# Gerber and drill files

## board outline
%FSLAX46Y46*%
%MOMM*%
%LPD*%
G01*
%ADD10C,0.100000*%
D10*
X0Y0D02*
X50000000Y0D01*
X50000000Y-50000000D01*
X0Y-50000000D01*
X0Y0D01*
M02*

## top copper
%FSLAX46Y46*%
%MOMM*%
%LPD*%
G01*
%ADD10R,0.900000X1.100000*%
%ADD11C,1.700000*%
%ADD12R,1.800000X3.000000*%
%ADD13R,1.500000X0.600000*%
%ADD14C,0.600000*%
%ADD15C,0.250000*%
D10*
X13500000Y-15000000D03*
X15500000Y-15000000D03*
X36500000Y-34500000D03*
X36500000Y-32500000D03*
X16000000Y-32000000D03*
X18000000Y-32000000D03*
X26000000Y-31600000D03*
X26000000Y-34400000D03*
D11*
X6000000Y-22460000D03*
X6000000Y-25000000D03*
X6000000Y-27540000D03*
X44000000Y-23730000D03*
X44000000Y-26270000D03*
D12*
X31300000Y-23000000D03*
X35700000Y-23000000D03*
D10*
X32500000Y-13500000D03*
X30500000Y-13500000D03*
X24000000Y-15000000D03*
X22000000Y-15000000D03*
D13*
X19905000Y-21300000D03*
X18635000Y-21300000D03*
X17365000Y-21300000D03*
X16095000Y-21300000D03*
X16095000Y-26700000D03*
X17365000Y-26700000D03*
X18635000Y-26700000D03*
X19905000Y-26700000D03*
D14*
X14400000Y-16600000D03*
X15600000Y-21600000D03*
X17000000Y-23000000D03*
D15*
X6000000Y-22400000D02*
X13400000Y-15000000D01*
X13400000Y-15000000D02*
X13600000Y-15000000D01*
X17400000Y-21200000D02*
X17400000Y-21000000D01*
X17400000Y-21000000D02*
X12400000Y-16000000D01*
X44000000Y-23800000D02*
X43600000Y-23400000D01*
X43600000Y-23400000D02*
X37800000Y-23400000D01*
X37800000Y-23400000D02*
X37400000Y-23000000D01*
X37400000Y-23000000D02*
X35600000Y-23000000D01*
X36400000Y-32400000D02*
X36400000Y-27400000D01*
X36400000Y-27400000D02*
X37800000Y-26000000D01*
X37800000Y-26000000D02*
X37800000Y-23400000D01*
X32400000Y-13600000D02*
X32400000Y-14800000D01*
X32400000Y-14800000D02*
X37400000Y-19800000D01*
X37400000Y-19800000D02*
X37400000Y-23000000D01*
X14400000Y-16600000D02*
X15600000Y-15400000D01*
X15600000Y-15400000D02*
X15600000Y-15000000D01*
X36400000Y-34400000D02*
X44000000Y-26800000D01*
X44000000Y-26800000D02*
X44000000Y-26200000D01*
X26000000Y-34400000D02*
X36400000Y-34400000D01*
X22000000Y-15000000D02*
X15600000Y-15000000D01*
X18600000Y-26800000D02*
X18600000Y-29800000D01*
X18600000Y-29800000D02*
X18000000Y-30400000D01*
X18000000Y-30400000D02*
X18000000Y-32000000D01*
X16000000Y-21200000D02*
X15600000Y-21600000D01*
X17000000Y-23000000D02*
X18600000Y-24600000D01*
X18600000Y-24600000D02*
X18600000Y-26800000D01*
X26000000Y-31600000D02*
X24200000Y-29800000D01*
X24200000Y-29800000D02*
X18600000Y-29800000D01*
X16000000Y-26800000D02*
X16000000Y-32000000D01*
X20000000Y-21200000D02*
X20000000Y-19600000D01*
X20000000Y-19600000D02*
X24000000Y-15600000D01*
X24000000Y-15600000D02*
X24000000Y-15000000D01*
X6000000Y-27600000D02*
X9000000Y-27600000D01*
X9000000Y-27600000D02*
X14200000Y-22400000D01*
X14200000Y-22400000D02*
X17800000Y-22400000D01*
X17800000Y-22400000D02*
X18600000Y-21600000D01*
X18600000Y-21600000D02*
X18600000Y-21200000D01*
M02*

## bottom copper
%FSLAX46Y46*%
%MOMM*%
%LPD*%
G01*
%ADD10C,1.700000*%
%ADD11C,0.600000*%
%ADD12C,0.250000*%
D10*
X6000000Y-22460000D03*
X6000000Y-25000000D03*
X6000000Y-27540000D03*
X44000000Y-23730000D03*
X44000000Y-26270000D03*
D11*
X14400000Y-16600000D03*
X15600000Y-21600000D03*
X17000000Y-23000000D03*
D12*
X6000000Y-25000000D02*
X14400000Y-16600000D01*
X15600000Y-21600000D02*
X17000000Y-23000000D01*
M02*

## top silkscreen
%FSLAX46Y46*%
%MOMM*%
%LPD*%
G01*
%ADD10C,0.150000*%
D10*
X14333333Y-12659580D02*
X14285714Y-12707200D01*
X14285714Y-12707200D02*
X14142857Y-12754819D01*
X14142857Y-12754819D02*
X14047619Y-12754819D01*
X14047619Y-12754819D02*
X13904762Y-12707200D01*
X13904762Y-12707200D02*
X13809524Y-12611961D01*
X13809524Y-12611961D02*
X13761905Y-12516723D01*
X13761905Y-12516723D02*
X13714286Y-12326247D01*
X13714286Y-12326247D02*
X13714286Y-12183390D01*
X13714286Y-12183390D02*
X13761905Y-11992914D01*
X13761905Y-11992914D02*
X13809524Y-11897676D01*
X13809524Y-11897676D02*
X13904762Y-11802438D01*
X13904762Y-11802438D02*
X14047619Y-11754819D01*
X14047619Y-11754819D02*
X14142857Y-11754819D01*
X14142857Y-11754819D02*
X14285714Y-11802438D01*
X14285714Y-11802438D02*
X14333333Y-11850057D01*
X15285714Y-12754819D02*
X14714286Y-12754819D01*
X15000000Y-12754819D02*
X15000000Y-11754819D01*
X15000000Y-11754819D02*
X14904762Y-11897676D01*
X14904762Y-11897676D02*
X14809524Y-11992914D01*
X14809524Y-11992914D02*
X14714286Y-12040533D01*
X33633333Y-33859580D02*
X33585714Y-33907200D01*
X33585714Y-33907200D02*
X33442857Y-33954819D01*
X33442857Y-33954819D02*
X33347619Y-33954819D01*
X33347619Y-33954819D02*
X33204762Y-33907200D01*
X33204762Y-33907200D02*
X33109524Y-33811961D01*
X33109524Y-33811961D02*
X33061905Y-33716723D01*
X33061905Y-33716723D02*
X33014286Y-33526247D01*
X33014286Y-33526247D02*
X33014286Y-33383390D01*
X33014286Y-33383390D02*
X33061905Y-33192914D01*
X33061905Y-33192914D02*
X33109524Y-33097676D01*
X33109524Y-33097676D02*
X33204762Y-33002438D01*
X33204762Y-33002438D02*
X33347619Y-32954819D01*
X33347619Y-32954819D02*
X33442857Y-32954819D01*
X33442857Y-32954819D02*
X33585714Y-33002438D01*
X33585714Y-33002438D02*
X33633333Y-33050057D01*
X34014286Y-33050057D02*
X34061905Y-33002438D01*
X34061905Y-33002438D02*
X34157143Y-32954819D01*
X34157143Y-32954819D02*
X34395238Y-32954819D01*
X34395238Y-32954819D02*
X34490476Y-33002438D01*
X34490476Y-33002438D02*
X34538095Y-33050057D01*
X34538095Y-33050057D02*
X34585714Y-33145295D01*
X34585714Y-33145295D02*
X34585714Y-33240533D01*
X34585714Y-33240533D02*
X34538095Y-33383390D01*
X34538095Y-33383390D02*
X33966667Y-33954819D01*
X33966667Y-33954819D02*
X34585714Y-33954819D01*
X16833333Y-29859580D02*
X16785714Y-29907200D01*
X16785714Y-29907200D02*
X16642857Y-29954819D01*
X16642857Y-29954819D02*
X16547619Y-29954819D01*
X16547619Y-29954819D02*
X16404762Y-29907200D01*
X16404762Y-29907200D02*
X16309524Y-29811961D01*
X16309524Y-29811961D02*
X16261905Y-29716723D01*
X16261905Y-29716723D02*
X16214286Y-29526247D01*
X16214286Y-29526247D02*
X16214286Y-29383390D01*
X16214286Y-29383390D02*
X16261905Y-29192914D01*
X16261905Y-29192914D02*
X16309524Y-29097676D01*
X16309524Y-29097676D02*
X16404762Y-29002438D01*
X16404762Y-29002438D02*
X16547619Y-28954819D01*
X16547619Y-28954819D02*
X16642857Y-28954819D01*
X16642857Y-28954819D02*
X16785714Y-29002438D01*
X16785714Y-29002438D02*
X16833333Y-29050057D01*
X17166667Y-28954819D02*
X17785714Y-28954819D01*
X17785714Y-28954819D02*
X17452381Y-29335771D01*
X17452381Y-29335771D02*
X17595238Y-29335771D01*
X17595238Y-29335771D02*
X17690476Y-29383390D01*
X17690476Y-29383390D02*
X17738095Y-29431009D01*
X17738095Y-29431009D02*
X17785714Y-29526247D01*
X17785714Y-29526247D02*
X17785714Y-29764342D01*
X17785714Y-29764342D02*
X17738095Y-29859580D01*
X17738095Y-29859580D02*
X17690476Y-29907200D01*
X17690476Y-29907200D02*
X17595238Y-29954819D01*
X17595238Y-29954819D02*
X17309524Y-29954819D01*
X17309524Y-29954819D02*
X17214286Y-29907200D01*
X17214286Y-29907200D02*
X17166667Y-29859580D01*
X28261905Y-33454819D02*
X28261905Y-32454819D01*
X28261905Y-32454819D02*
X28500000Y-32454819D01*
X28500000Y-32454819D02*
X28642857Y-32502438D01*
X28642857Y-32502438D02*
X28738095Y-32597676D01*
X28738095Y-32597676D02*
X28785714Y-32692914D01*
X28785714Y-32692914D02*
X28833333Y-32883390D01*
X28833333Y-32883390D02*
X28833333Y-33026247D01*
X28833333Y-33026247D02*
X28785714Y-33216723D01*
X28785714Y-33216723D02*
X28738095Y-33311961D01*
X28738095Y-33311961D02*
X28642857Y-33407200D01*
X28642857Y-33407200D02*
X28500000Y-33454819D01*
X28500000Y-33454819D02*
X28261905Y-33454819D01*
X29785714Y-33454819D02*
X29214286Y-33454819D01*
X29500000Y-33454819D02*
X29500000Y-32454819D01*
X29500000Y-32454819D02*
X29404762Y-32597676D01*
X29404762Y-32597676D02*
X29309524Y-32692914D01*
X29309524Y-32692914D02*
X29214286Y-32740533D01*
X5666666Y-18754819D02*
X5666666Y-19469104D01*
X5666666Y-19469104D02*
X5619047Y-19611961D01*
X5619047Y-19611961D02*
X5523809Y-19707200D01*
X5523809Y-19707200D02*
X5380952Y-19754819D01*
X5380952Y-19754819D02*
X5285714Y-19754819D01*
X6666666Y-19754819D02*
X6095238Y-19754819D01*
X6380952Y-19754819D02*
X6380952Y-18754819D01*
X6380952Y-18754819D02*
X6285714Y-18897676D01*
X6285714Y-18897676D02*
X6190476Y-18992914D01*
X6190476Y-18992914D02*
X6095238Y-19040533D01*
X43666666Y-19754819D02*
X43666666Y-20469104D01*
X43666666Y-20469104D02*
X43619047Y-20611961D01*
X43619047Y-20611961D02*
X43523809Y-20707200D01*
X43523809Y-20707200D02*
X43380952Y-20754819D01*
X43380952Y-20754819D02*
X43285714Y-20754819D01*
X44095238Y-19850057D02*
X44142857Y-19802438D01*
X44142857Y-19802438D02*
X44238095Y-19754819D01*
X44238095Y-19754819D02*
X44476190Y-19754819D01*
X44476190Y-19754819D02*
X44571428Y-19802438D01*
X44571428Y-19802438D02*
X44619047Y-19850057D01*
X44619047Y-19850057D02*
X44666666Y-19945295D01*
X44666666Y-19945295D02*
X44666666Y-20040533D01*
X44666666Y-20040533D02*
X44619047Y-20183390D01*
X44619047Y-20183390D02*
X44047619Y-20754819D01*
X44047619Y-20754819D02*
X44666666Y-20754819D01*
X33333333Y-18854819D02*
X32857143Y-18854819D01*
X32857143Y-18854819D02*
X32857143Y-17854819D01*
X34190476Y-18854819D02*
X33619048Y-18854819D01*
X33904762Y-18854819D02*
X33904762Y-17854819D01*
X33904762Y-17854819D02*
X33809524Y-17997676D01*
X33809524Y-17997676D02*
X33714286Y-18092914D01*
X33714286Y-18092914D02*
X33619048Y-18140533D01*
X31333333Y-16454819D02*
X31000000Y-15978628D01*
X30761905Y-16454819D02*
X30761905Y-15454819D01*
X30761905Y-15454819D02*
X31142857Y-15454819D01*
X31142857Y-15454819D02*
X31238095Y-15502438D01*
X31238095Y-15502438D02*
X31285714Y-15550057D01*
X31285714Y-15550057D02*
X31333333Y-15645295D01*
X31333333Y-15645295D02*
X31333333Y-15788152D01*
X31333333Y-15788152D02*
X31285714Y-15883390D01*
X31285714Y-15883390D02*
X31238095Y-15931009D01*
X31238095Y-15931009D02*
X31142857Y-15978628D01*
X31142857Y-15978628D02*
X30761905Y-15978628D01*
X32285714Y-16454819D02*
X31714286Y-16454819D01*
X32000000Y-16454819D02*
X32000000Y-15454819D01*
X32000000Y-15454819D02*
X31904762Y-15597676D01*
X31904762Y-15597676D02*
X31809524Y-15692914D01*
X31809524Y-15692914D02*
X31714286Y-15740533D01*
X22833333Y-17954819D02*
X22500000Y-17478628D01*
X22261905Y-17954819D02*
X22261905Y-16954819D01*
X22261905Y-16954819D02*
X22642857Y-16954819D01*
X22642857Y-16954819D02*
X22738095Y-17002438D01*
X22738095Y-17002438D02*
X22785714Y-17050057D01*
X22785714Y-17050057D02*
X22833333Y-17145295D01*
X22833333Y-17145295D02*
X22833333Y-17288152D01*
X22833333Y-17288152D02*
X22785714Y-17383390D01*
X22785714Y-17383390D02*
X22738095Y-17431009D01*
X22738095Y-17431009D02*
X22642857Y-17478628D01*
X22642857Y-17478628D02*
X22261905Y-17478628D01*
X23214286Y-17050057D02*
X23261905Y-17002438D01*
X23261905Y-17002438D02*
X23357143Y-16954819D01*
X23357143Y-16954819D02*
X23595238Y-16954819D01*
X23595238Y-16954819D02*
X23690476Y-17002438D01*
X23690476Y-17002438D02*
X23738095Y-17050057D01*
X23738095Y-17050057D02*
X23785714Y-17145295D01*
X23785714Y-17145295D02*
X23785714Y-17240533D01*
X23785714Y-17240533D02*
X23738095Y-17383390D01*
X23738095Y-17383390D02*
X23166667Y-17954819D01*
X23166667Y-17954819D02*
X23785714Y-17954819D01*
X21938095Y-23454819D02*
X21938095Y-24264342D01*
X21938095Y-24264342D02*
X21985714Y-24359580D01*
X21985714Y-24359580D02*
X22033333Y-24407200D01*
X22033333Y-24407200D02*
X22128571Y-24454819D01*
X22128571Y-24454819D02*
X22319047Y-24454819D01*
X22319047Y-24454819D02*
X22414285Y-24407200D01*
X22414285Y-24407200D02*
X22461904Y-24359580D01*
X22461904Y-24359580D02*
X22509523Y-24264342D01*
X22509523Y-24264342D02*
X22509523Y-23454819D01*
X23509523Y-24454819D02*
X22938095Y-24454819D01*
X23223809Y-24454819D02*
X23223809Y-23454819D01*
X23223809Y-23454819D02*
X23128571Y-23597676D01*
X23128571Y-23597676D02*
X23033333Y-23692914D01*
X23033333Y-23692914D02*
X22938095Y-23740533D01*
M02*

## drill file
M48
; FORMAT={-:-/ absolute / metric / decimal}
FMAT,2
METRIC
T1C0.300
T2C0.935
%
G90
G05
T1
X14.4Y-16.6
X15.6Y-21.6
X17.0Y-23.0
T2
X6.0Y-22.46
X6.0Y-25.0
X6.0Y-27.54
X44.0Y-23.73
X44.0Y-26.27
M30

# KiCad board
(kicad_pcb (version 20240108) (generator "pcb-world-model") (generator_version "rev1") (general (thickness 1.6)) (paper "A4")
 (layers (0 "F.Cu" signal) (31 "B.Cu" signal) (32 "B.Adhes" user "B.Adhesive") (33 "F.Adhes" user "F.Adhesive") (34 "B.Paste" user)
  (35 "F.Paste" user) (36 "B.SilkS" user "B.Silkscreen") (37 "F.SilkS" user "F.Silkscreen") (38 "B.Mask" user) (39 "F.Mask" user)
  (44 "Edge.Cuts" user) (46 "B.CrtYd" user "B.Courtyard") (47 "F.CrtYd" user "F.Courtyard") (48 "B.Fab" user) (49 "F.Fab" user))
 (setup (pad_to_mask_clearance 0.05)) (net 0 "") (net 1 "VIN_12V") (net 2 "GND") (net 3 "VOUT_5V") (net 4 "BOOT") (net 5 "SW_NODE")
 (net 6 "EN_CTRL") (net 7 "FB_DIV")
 (gr_rect (start 0.0 0.0) (end 50.0000 50.0000) (stroke (width 0.1) (type default)) (fill none) (layer "Edge.Cuts"))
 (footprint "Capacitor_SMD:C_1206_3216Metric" (layer "F.Cu") (at 14.5000 15.0000 0)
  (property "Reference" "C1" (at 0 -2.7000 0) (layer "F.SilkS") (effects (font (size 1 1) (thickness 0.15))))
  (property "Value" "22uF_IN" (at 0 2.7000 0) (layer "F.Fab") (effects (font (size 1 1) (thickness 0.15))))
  (pad "1" smd rect (at -1.0000 0.0000) (size 0.9000 1.1000) (layers "F.Cu" "F.Paste" "F.Mask") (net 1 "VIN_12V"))
  (pad "2" smd rect (at 1.0000 0.0000) (size 0.9000 1.1000) (layers "F.Cu" "F.Paste" "F.Mask") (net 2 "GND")))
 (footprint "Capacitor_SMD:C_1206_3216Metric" (layer "F.Cu") (at 36.5000 33.5000 90)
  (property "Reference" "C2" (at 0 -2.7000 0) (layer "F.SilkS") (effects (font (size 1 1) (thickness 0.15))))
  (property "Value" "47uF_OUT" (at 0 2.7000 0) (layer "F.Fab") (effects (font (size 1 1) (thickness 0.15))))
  (pad "1" smd rect (at -1.0000 0.0000) (size 0.9000 1.1000) (layers "F.Cu" "F.Paste" "F.Mask") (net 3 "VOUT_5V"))
  (pad "2" smd rect (at 1.0000 0.0000) (size 0.9000 1.1000) (layers "F.Cu" "F.Paste" "F.Mask") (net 2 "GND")))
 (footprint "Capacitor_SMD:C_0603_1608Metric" (layer "F.Cu") (at 17.0000 32.0000 0)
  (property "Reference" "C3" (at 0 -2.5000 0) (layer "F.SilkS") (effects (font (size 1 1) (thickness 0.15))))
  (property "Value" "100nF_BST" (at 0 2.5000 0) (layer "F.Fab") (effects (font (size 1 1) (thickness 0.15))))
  (pad "1" smd rect (at -1.0000 0.0000) (size 0.9000 1.1000) (layers "F.Cu" "F.Paste" "F.Mask") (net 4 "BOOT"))
  (pad "2" smd rect (at 1.0000 0.0000) (size 0.9000 1.1000) (layers "F.Cu" "F.Paste" "F.Mask") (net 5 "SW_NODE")))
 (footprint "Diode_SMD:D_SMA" (layer "F.Cu") (at 26.0000 33.0000 270)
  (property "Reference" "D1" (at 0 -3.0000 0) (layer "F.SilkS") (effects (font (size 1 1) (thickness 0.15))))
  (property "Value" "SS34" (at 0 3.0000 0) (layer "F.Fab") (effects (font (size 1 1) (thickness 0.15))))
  (pad "1" smd rect (at -1.4000 0.0000) (size 0.9000 1.1000) (layers "F.Cu" "F.Paste" "F.Mask") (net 2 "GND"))
  (pad "2" smd rect (at 1.4000 0.0000) (size 0.9000 1.1000) (layers "F.Cu" "F.Paste" "F.Mask") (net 5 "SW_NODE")))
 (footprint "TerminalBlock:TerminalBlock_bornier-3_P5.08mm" (layer "F.Cu") (at 6.0000 25.0000 0) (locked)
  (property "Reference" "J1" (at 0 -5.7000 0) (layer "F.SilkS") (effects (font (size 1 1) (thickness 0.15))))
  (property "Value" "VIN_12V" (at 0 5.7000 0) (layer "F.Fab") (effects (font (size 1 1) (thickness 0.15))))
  (pad "1" thru_hole circle (at 0.0000 -2.5400) (size 1.7000 1.7000) (drill 0.9350) (layers "*.Cu" "*.Mask") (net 1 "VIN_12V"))
  (pad "2" thru_hole circle (at 0.0000 0.0000) (size 1.7000 1.7000) (drill 0.9350) (layers "*.Cu" "*.Mask") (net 2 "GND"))
  (pad "3" thru_hole circle (at 0.0000 2.5400) (size 1.7000 1.7000) (drill 0.9350) (layers "*.Cu" "*.Mask") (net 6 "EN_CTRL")))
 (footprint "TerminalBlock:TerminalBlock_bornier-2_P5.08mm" (layer "F.Cu") (at 44.0000 25.0000 0) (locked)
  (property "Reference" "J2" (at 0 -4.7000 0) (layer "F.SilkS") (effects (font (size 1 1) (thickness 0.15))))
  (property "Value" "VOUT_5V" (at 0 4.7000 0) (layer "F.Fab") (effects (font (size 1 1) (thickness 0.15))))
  (pad "1" thru_hole circle (at 0.0000 -1.2700) (size 1.7000 1.7000) (drill 0.9350) (layers "*.Cu" "*.Mask") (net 3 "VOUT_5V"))
  (pad "2" thru_hole circle (at 0.0000 1.2700) (size 1.7000 1.7000) (drill 0.9350) (layers "*.Cu" "*.Mask") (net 2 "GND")))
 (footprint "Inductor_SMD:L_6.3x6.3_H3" (layer "F.Cu") (at 33.5000 23.0000 0)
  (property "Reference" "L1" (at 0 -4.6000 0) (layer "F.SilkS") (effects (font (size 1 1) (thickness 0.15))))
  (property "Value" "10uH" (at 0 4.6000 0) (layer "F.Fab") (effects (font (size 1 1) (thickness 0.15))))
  (pad "1" smd rect (at -2.2000 0.0000) (size 1.8000 3.0000) (layers "F.Cu" "F.Paste" "F.Mask") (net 5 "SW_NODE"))
  (pad "2" smd rect (at 2.2000 0.0000) (size 1.8000 3.0000) (layers "F.Cu" "F.Paste" "F.Mask") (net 3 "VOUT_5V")))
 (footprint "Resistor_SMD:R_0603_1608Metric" (layer "F.Cu") (at 31.5000 13.5000 180)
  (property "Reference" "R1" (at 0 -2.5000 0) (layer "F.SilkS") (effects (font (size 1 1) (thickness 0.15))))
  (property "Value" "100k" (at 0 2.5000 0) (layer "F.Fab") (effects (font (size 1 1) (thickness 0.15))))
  (pad "1" smd rect (at -1.0000 0.0000) (size 0.9000 1.1000) (layers "F.Cu" "F.Paste" "F.Mask") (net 3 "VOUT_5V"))
  (pad "2" smd rect (at 1.0000 0.0000) (size 0.9000 1.1000) (layers "F.Cu" "F.Paste" "F.Mask") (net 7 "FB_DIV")))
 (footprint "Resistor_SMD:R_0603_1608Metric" (layer "F.Cu") (at 23.0000 15.0000 180)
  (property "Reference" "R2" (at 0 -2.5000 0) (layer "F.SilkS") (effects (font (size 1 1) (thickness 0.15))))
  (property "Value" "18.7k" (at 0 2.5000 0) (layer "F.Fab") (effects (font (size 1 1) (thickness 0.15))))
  (pad "1" smd rect (at -1.0000 0.0000) (size 0.9000 1.1000) (layers "F.Cu" "F.Paste" "F.Mask") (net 7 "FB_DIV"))
  (pad "2" smd rect (at 1.0000 0.0000) (size 0.9000 1.1000) (layers "F.Cu" "F.Paste" "F.Mask") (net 2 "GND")))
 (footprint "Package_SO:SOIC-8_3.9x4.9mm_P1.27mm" (layer "F.Cu") (at 18.0000 24.0000 270)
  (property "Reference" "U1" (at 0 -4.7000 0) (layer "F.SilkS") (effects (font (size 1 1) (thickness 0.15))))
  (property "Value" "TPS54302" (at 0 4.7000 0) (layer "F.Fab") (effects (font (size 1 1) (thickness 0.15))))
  (pad "1" smd rect (at -2.7000 -1.9050) (size 1.5000 0.6000) (layers "F.Cu" "F.Paste" "F.Mask") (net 4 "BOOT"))
  (pad "2" smd rect (at -2.7000 -0.6350) (size 1.5000 0.6000) (layers "F.Cu" "F.Paste" "F.Mask") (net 1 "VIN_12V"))
  (pad "3" smd rect (at -2.7000 0.6350) (size 1.5000 0.6000) (layers "F.Cu" "F.Paste" "F.Mask") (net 5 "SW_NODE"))
  (pad "4" smd rect (at -2.7000 1.9050) (size 1.5000 0.6000) (layers "F.Cu" "F.Paste" "F.Mask") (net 2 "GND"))
  (pad "5" smd rect (at 2.7000 1.9050) (size 1.5000 0.6000) (layers "F.Cu" "F.Paste" "F.Mask") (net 7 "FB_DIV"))
  (pad "6" smd rect (at 2.7000 0.6350) (size 1.5000 0.6000) (layers "F.Cu" "F.Paste" "F.Mask") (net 6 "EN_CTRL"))
  (pad "7" smd rect (at 2.7000 -0.6350) (size 1.5000 0.6000) (layers "F.Cu" "F.Paste" "F.Mask") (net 1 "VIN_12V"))
  (pad "8" smd rect (at 2.7000 -1.9050) (size 1.5000 0.6000) (layers "F.Cu" "F.Paste" "F.Mask") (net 5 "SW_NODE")))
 (segment (start 6.0000 22.4000) (end 13.4000 15.0000) (width 0.2500) (layer "F.Cu") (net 1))
 (segment (start 13.4000 15.0000) (end 13.6000 15.0000) (width 0.2500) (layer "F.Cu") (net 1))
 (segment (start 17.4000 21.2000) (end 17.4000 21.0000) (width 0.2500) (layer "F.Cu") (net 1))
 (segment (start 17.4000 21.0000) (end 12.4000 16.0000) (width 0.2500) (layer "F.Cu") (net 1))
 (segment (start 44.0000 23.8000) (end 43.6000 23.4000) (width 0.2500) (layer "F.Cu") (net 3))
 (segment (start 43.6000 23.4000) (end 37.8000 23.4000) (width 0.2500) (layer "F.Cu") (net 3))
 (segment (start 37.8000 23.4000) (end 37.4000 23.0000) (width 0.2500) (layer "F.Cu") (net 3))
 (segment (start 37.4000 23.0000) (end 35.6000 23.0000) (width 0.2500) (layer "F.Cu") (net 3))
 (segment (start 36.4000 32.4000) (end 36.4000 27.4000) (width 0.2500) (layer "F.Cu") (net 3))
 (segment (start 36.4000 27.4000) (end 37.8000 26.0000) (width 0.2500) (layer "F.Cu") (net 3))
 (segment (start 37.8000 26.0000) (end 37.8000 23.4000) (width 0.2500) (layer "F.Cu") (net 3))
 (segment (start 32.4000 13.6000) (end 32.4000 14.8000) (width 0.2500) (layer "F.Cu") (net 3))
 (segment (start 32.4000 14.8000) (end 37.4000 19.8000) (width 0.2500) (layer "F.Cu") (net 3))
 (segment (start 37.4000 19.8000) (end 37.4000 23.0000) (width 0.2500) (layer "F.Cu") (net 3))
 (segment (start 6.0000 25.0000) (end 14.4000 16.6000) (width 0.2500) (layer "B.Cu") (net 2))
 (segment (start 14.4000 16.6000) (end 15.6000 15.4000) (width 0.2500) (layer "F.Cu") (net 2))
 (segment (start 15.6000 15.4000) (end 15.6000 15.0000) (width 0.2500) (layer "F.Cu") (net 2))
 (segment (start 36.4000 34.4000) (end 44.0000 26.8000) (width 0.2500) (layer "F.Cu") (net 2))
 (segment (start 44.0000 26.8000) (end 44.0000 26.2000) (width 0.2500) (layer "F.Cu") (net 2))
 (segment (start 26.0000 34.4000) (end 36.4000 34.4000) (width 0.2500) (layer "F.Cu") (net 2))
 (segment (start 22.0000 15.0000) (end 15.6000 15.0000) (width 0.2500) (layer "F.Cu") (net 2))
 (segment (start 18.6000 26.8000) (end 18.6000 29.8000) (width 0.2500) (layer "F.Cu") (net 5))
 (segment (start 18.6000 29.8000) (end 18.0000 30.4000) (width 0.2500) (layer "F.Cu") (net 5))
 (segment (start 18.0000 30.4000) (end 18.0000 32.0000) (width 0.2500) (layer "F.Cu") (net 5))
 (segment (start 16.0000 21.2000) (end 15.6000 21.6000) (width 0.2500) (layer "F.Cu") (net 5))
 (segment (start 15.6000 21.6000) (end 17.0000 23.0000) (width 0.2500) (layer "B.Cu") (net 5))
 (segment (start 17.0000 23.0000) (end 18.6000 24.6000) (width 0.2500) (layer "F.Cu") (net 5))
 (segment (start 18.6000 24.6000) (end 18.6000 26.8000) (width 0.2500) (layer "F.Cu") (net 5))
 (segment (start 26.0000 31.6000) (end 24.2000 29.8000) (width 0.2500) (layer "F.Cu") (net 5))
 (segment (start 24.2000 29.8000) (end 18.6000 29.8000) (width 0.2500) (layer "F.Cu") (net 5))
 (segment (start 16.0000 26.8000) (end 16.0000 32.0000) (width 0.2500) (layer "F.Cu") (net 4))
 (segment (start 20.0000 21.2000) (end 20.0000 19.6000) (width 0.2500) (layer "F.Cu") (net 7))
 (segment (start 20.0000 19.6000) (end 24.0000 15.6000) (width 0.2500) (layer "F.Cu") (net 7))
 (segment (start 24.0000 15.6000) (end 24.0000 15.0000) (width 0.2500) (layer "F.Cu") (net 7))
 (segment (start 6.0000 27.6000) (end 9.0000 27.6000) (width 0.2500) (layer "F.Cu") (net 6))
 (segment (start 9.0000 27.6000) (end 14.2000 22.4000) (width 0.2500) (layer "F.Cu") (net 6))
 (segment (start 14.2000 22.4000) (end 17.8000 22.4000) (width 0.2500) (layer "F.Cu") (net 6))
 (segment (start 17.8000 22.4000) (end 18.6000 21.6000) (width 0.2500) (layer "F.Cu") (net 6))
 (segment (start 18.6000 21.6000) (end 18.6000 21.2000) (width 0.2500) (layer "F.Cu") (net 6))
 (via (at 14.4000 16.6000) (size 0.6000) (drill 0.3000) (layers "F.Cu" "B.Cu") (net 2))
 (via (at 15.6000 21.6000) (size 0.6000) (drill 0.3000) (layers "F.Cu" "B.Cu") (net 5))
 (via (at 17.0000 23.0000) (size 0.6000) (drill 0.3000) (layers "F.Cu" "B.Cu") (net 5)))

